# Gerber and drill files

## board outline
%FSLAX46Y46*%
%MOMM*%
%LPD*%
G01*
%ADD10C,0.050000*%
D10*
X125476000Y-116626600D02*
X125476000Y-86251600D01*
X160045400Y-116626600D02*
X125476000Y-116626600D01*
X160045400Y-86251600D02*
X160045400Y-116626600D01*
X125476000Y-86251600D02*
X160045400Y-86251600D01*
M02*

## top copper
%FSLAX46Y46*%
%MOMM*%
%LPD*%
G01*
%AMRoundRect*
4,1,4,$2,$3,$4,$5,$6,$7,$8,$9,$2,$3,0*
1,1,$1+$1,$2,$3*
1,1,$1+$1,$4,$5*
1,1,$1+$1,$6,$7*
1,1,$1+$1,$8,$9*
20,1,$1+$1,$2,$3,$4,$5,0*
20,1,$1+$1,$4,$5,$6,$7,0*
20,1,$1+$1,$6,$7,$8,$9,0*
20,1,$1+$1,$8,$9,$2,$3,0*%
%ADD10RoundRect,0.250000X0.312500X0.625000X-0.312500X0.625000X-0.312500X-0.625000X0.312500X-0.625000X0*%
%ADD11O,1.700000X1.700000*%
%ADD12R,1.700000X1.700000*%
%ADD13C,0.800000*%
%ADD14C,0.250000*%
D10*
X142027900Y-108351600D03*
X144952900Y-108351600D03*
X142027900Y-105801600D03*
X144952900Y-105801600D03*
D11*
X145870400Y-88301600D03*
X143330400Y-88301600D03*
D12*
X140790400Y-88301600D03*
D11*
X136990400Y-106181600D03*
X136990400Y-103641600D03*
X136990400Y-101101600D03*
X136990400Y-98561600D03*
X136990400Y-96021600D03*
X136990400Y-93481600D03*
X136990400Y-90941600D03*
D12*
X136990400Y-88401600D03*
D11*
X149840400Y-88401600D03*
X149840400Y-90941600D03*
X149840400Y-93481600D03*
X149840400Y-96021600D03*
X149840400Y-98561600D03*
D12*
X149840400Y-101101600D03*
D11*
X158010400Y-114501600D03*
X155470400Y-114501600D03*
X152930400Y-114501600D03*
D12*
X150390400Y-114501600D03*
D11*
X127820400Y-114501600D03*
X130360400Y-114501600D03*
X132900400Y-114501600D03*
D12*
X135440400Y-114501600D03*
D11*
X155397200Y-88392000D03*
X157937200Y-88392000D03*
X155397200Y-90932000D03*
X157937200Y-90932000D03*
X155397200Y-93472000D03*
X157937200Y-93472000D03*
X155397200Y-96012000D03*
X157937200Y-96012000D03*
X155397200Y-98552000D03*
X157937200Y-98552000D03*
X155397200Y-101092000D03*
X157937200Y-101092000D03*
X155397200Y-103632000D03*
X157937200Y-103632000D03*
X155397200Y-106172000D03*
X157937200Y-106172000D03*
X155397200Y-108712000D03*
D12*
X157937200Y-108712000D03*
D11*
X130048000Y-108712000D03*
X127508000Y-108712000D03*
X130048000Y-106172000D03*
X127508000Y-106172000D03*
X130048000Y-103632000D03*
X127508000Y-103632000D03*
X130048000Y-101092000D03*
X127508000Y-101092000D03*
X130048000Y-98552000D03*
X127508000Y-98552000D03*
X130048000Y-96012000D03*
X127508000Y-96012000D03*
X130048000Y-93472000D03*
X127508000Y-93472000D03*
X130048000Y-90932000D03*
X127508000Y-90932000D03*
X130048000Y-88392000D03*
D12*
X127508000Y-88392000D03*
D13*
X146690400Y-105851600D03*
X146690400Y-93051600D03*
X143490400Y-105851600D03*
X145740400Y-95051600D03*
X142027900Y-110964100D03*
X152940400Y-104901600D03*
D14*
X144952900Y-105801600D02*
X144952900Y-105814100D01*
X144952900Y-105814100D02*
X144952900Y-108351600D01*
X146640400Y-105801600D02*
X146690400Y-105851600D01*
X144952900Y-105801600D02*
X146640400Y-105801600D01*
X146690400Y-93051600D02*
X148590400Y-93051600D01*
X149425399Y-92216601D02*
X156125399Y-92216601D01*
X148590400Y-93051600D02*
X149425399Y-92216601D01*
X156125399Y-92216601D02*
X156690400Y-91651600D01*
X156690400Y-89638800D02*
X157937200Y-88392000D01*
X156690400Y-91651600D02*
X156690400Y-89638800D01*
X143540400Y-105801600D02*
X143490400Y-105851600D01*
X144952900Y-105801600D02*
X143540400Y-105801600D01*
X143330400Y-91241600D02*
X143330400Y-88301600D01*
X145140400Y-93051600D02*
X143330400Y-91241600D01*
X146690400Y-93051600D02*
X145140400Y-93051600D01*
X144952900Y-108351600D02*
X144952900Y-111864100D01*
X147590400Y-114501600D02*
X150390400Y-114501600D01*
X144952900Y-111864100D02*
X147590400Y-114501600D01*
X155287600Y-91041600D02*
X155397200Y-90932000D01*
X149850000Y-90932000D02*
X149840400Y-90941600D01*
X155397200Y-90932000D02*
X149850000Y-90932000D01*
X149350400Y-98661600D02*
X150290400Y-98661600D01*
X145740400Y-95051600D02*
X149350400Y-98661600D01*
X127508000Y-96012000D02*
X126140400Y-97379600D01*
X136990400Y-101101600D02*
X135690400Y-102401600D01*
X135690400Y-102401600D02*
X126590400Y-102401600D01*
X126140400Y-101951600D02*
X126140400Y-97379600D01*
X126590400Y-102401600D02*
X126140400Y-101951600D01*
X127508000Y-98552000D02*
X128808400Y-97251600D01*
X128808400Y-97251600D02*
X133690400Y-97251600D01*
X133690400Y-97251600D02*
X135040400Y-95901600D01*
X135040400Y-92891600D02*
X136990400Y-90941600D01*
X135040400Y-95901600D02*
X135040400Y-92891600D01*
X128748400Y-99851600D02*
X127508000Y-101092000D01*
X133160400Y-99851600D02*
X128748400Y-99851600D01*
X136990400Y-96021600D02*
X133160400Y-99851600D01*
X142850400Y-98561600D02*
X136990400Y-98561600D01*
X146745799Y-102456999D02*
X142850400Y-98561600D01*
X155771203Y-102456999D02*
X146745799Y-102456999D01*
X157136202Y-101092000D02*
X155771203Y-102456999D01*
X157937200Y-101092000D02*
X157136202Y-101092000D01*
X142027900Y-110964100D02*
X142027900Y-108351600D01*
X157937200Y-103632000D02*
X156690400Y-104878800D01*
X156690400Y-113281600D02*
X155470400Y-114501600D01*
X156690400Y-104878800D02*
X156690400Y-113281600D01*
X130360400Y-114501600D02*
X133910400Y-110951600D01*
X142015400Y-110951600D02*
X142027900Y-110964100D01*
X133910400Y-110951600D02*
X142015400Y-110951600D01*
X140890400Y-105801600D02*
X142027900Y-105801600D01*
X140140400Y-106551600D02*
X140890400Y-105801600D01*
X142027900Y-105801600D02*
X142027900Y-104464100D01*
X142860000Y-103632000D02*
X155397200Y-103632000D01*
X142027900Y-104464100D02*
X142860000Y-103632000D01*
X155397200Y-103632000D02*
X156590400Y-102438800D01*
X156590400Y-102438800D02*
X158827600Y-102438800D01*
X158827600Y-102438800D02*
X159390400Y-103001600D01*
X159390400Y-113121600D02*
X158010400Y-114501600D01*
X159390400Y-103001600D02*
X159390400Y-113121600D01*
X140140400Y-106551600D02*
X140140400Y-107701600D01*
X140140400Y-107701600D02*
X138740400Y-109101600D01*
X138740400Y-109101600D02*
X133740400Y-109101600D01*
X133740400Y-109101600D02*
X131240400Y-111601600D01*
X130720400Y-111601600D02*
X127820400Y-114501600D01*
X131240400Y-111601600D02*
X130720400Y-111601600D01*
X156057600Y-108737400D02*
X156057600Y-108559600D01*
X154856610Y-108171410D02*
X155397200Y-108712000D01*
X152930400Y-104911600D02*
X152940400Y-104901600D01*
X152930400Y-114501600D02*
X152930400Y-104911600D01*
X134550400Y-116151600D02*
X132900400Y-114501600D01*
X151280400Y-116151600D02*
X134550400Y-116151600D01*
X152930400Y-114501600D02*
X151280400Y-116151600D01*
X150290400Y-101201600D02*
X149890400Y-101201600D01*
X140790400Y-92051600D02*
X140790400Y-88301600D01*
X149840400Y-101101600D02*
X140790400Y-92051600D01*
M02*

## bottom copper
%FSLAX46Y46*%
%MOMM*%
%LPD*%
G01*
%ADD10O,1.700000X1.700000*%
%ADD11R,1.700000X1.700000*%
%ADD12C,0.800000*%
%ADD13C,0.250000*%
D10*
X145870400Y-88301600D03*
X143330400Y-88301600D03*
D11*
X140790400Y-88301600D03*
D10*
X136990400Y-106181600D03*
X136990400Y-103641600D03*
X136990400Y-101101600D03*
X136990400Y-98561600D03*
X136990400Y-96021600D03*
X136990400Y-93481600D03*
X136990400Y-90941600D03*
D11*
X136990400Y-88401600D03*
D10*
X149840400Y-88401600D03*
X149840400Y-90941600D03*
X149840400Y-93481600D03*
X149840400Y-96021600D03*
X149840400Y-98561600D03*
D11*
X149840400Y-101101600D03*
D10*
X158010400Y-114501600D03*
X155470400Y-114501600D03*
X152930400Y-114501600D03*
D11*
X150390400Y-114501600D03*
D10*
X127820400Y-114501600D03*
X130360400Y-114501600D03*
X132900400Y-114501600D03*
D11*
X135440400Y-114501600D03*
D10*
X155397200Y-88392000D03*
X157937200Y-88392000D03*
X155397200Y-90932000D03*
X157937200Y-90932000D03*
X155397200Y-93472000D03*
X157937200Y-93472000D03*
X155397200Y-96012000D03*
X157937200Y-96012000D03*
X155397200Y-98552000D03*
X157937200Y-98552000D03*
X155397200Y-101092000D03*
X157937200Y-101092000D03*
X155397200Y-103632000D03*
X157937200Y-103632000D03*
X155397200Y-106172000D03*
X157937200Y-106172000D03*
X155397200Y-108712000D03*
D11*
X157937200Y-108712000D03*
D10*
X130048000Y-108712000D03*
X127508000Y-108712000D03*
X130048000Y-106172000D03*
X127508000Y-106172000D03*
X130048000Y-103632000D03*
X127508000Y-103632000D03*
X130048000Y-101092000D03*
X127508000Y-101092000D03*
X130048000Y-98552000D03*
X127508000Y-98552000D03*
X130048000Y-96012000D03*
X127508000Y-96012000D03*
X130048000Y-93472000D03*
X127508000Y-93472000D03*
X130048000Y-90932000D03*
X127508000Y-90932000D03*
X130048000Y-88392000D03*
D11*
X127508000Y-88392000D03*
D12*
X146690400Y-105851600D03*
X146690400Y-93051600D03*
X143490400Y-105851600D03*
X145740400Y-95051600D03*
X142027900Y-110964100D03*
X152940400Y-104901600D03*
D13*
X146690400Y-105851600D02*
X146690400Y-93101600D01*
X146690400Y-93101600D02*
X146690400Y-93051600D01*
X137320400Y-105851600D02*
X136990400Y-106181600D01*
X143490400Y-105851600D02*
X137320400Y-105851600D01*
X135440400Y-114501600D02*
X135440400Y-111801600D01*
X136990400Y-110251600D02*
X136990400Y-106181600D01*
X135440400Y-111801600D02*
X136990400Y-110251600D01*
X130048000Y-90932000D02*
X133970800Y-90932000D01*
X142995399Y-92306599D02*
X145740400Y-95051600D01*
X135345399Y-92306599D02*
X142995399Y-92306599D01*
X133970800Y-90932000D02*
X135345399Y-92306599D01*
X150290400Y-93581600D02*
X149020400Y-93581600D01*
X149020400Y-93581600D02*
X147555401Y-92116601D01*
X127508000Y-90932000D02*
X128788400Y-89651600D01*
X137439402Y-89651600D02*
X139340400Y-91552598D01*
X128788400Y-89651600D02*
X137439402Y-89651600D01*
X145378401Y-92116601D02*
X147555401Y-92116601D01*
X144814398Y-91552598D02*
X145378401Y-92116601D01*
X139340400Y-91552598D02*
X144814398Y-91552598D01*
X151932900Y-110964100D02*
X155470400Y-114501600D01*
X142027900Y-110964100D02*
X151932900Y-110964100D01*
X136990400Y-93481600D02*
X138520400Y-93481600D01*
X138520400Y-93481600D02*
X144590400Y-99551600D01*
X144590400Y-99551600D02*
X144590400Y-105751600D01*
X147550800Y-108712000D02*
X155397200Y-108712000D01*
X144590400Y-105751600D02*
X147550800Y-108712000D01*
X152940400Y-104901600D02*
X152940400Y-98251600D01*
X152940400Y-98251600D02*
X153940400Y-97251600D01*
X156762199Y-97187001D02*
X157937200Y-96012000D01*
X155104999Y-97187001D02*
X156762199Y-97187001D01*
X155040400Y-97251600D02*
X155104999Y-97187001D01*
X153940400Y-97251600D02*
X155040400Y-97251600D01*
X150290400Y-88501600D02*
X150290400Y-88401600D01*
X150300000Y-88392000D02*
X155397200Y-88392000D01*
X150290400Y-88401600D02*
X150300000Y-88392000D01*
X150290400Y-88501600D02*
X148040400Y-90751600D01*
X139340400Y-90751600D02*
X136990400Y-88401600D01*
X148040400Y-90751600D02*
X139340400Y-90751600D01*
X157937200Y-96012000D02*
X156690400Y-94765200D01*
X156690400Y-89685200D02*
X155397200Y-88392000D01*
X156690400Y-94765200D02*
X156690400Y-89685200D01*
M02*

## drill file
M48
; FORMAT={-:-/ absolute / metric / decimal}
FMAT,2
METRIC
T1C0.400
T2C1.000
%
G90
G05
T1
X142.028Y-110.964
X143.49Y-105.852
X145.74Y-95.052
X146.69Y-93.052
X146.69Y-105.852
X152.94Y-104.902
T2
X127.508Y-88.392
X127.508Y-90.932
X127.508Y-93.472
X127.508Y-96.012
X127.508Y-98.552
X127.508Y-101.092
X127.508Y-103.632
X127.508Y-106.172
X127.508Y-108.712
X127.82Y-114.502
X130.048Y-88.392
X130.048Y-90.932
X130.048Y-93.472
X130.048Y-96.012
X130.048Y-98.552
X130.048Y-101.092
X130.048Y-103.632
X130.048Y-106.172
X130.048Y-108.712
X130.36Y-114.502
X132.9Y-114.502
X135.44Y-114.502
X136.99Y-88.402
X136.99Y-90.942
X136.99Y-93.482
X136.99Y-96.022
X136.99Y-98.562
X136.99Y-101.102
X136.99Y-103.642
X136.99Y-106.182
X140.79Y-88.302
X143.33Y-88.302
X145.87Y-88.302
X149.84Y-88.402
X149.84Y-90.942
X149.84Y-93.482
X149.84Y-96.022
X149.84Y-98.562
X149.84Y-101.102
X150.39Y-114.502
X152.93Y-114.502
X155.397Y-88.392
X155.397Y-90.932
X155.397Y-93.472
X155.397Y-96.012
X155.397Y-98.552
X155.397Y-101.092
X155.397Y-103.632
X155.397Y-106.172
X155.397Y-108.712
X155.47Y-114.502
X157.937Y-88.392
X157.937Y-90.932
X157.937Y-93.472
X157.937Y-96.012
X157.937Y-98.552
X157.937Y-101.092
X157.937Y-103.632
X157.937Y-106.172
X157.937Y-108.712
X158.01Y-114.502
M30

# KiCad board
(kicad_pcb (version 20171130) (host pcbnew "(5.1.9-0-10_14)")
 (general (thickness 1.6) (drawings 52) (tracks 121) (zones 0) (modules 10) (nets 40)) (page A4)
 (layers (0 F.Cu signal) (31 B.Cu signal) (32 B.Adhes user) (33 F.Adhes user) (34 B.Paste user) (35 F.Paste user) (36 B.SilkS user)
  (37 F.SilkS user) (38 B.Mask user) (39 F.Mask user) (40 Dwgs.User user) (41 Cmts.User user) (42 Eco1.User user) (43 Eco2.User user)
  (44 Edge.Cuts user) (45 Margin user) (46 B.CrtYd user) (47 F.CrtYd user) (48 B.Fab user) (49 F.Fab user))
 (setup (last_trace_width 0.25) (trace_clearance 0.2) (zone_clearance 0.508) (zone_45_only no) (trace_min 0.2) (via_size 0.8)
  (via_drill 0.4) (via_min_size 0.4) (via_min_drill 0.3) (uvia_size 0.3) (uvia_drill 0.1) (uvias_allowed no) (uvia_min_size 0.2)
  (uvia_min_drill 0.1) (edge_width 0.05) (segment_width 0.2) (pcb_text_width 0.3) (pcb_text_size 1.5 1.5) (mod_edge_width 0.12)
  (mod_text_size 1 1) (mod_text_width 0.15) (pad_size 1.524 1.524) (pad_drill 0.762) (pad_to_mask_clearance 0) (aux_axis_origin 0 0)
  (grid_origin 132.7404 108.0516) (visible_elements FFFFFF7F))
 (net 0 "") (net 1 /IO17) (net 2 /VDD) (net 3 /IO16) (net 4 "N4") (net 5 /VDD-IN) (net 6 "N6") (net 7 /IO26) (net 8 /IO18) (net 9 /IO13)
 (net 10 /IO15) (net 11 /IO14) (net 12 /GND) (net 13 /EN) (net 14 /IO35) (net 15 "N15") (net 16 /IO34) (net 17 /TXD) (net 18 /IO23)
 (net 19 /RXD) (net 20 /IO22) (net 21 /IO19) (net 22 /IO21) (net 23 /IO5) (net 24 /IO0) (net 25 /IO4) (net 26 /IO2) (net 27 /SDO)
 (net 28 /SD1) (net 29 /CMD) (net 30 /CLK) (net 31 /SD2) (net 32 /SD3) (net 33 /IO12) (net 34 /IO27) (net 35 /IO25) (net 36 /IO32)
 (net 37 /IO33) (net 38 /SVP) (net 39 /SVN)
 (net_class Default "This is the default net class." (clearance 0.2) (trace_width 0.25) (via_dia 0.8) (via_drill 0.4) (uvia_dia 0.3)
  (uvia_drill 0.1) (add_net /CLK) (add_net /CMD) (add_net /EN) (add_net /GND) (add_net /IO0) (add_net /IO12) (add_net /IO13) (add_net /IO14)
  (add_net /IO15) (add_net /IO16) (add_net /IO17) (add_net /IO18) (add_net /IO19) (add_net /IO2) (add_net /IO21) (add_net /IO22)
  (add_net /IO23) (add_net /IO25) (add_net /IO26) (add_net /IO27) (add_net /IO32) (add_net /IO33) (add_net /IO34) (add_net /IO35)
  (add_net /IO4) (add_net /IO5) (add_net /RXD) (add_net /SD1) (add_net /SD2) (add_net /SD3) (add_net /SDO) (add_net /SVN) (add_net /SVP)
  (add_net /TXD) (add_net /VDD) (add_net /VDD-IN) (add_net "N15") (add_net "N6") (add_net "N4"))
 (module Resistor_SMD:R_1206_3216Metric (layer F.Cu) (at 143.4904 108.3516 180)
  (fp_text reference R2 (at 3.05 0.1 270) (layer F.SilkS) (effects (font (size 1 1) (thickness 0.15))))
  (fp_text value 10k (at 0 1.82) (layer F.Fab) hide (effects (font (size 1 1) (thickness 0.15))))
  (pad 2 smd roundrect (at 1.4625 0 180) (size 1.125 1.75) (layers F.Cu F.Paste F.Mask) (roundrect_rratio 0.222222) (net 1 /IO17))
  (pad 1 smd roundrect (at -1.4625 0 180) (size 1.125 1.75) (layers F.Cu F.Paste F.Mask) (roundrect_rratio 0.222222) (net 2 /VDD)))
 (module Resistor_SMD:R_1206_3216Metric (layer F.Cu) (at 143.4904 105.8016 180)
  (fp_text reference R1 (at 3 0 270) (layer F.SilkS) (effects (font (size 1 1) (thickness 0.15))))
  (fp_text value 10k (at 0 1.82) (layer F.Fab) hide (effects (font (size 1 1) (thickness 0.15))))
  (pad 2 smd roundrect (at 1.4625 0 180) (size 1.125 1.75) (layers F.Cu F.Paste F.Mask) (roundrect_rratio 0.222222) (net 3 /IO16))
  (pad 1 smd roundrect (at -1.4625 0 180) (size 1.125 1.75) (layers F.Cu F.Paste F.Mask) (roundrect_rratio 0.222222) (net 2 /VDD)))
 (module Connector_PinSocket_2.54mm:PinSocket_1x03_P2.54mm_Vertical (layer B.Cu) (at 140.7904 88.3016 270)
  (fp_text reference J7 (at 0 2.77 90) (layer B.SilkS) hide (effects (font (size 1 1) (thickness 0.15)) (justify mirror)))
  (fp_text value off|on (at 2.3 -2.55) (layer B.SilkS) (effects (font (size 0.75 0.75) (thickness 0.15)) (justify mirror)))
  (pad 3 thru_hole oval (at 0 -5.08 270) (size 1.7 1.7) (drill 1) (layers *.Cu *.Mask) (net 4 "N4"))
  (pad 2 thru_hole oval (at 0 -2.54 270) (size 1.7 1.7) (drill 1) (layers *.Cu *.Mask) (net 2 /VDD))
  (pad 1 thru_hole rect (at 0 0 270) (size 1.7 1.7) (drill 1) (layers *.Cu *.Mask) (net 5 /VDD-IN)))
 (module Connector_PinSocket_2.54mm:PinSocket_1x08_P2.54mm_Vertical (layer B.Cu) (at 136.9904 88.4016 180)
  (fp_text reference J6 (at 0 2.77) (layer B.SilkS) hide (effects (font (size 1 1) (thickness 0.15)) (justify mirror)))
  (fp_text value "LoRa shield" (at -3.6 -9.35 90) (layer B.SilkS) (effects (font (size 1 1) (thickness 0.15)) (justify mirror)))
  (pad 8 thru_hole oval (at 0 -17.78 180) (size 1.7 1.7) (drill 1) (layers *.Cu *.Mask) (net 2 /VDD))
  (pad 7 thru_hole oval (at 0 -15.24 180) (size 1.7 1.7) (drill 1) (layers *.Cu *.Mask) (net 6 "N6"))
  (pad 6 thru_hole oval (at 0 -12.7 180) (size 1.7 1.7) (drill 1) (layers *.Cu *.Mask) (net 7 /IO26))
  (pad 5 thru_hole oval (at 0 -10.16 180) (size 1.7 1.7) (drill 1) (layers *.Cu *.Mask) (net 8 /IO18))
  (pad 4 thru_hole oval (at 0 -7.62 180) (size 1.7 1.7) (drill 1) (layers *.Cu *.Mask) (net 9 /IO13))
  (pad 3 thru_hole oval (at 0 -5.08 180) (size 1.7 1.7) (drill 1) (layers *.Cu *.Mask) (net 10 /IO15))
  (pad 2 thru_hole oval (at 0 -2.54 180) (size 1.7 1.7) (drill 1) (layers *.Cu *.Mask) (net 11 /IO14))
  (pad 1 thru_hole rect (at 0 0 180) (size 1.7 1.7) (drill 1) (layers *.Cu *.Mask) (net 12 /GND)))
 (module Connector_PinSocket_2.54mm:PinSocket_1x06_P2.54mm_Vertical (layer B.Cu) (at 149.8404 101.1016)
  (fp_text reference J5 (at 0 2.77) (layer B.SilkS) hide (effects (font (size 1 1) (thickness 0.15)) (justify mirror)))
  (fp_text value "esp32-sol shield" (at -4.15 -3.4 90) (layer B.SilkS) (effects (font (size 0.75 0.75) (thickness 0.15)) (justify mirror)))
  (pad 6 thru_hole oval (at 0 -12.7) (size 1.7 1.7) (drill 1) (layers *.Cu *.Mask) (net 12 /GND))
  (pad 5 thru_hole oval (at 0 -10.16) (size 1.7 1.7) (drill 1) (layers *.Cu *.Mask) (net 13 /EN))
  (pad 4 thru_hole oval (at 0 -7.62) (size 1.7 1.7) (drill 1) (layers *.Cu *.Mask) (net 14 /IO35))
  (pad 3 thru_hole oval (at 0 -5.08) (size 1.7 1.7) (drill 1) (layers *.Cu *.Mask) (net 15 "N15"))
  (pad 2 thru_hole oval (at 0 -2.54) (size 1.7 1.7) (drill 1) (layers *.Cu *.Mask) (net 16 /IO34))
  (pad 1 thru_hole rect (at 0 0) (size 1.7 1.7) (drill 1) (layers *.Cu *.Mask) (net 5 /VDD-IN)))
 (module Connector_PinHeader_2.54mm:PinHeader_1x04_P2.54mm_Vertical (layer B.Cu) (at 150.3904 114.5016 270)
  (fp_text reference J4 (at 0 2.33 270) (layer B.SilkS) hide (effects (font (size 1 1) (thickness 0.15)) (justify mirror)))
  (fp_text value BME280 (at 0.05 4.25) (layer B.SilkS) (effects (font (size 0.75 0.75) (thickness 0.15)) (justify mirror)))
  (pad 4 thru_hole oval (at 0 -7.62 270) (size 1.7 1.7) (drill 1) (layers *.Cu *.Mask) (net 3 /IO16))
  (pad 3 thru_hole oval (at 0 -5.08 270) (size 1.7 1.7) (drill 1) (layers *.Cu *.Mask) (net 1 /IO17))
  (pad 2 thru_hole oval (at 0 -2.54 270) (size 1.7 1.7) (drill 1) (layers *.Cu *.Mask) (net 12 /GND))
  (pad 1 thru_hole rect (at 0 0 270) (size 1.7 1.7) (drill 1) (layers *.Cu *.Mask) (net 2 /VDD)))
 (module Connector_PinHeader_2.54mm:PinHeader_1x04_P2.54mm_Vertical (layer B.Cu) (at 135.4404 114.5016 90)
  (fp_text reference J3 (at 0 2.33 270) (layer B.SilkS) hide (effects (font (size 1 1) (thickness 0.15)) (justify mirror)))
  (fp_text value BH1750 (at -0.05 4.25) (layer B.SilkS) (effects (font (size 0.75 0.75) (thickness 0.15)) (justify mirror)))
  (pad 4 thru_hole oval (at 0 -7.62 90) (size 1.7 1.7) (drill 1) (layers *.Cu *.Mask) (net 3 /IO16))
  (pad 3 thru_hole oval (at 0 -5.08 90) (size 1.7 1.7) (drill 1) (layers *.Cu *.Mask) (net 1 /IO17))
  (pad 2 thru_hole oval (at 0 -2.54 90) (size 1.7 1.7) (drill 1) (layers *.Cu *.Mask) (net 12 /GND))
  (pad 1 thru_hole rect (at 0 0 90) (size 1.7 1.7) (drill 1) (layers *.Cu *.Mask) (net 2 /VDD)))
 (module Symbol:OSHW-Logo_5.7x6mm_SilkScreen (layer F.Cu) (at 143.6404 94.9016)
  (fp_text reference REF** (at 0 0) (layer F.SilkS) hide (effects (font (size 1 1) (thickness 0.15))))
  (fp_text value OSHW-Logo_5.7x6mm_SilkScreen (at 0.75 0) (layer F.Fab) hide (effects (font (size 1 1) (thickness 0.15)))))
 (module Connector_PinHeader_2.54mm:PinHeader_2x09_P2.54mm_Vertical (layer F.Cu) (at 157.9372 108.712 180)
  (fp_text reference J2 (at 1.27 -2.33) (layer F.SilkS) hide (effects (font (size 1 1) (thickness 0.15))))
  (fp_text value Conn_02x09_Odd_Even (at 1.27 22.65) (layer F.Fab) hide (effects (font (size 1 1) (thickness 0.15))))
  (pad 18 thru_hole oval (at 2.54 20.32 180) (size 1.7 1.7) (drill 1) (layers *.Cu *.Mask) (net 12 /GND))
  (pad 17 thru_hole oval (at 0 20.32 180) (size 1.7 1.7) (drill 1) (layers *.Cu *.Mask) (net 2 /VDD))
  (pad 16 thru_hole oval (at 2.54 17.78 180) (size 1.7 1.7) (drill 1) (layers *.Cu *.Mask) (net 13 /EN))
  (pad 15 thru_hole oval (at 0 17.78 180) (size 1.7 1.7) (drill 1) (layers *.Cu *.Mask) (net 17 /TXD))
  (pad 14 thru_hole oval (at 2.54 15.24 180) (size 1.7 1.7) (drill 1) (layers *.Cu *.Mask) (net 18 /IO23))
  (pad 13 thru_hole oval (at 0 15.24 180) (size 1.7 1.7) (drill 1) (layers *.Cu *.Mask) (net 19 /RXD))
  (pad 12 thru_hole oval (at 2.54 12.7 180) (size 1.7 1.7) (drill 1) (layers *.Cu *.Mask) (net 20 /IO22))
  (pad 11 thru_hole oval (at 0 12.7 180) (size 1.7 1.7) (drill 1) (layers *.Cu *.Mask) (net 12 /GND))
  (pad 10 thru_hole oval (at 2.54 10.16 180) (size 1.7 1.7) (drill 1) (layers *.Cu *.Mask) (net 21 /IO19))
  (pad 9 thru_hole oval (at 0 10.16 180) (size 1.7 1.7) (drill 1) (layers *.Cu *.Mask) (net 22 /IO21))
  (pad 8 thru_hole oval (at 2.54 7.62 180) (size 1.7 1.7) (drill 1) (layers *.Cu *.Mask) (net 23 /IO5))
  (pad 7 thru_hole oval (at 0 7.62 180) (size 1.7 1.7) (drill 1) (layers *.Cu *.Mask) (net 8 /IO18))
  (pad 6 thru_hole oval (at 2.54 5.08 180) (size 1.7 1.7) (drill 1) (layers *.Cu *.Mask) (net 3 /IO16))
  (pad 5 thru_hole oval (at 0 5.08 180) (size 1.7 1.7) (drill 1) (layers *.Cu *.Mask) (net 1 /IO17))
  (pad 4 thru_hole oval (at 2.54 2.54 180) (size 1.7 1.7) (drill 1) (layers *.Cu *.Mask) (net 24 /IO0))
  (pad 3 thru_hole oval (at 0 2.54 180) (size 1.7 1.7) (drill 1) (layers *.Cu *.Mask) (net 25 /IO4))
  (pad 2 thru_hole oval (at 2.54 0 180) (size 1.7 1.7) (drill 1) (layers *.Cu *.Mask) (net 10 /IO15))
  (pad 1 thru_hole rect (at 0 0 180) (size 1.7 1.7) (drill 1) (layers *.Cu *.Mask) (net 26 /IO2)))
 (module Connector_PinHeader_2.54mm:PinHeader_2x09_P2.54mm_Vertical (layer F.Cu) (at 127.508 88.392)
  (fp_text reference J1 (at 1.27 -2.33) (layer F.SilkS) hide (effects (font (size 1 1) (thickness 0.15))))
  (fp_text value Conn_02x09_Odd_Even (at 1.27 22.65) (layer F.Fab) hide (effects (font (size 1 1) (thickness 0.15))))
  (pad 18 thru_hole oval (at 2.54 20.32) (size 1.7 1.7) (drill 1) (layers *.Cu *.Mask) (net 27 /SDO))
  (pad 17 thru_hole oval (at 0 20.32) (size 1.7 1.7) (drill 1) (layers *.Cu *.Mask) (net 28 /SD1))
  (pad 16 thru_hole oval (at 2.54 17.78) (size 1.7 1.7) (drill 1) (layers *.Cu *.Mask) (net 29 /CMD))
  (pad 15 thru_hole oval (at 0 17.78) (size 1.7 1.7) (drill 1) (layers *.Cu *.Mask) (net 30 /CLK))
  (pad 14 thru_hole oval (at 2.54 15.24) (size 1.7 1.7) (drill 1) (layers *.Cu *.Mask) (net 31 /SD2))
  (pad 13 thru_hole oval (at 0 15.24) (size 1.7 1.7) (drill 1) (layers *.Cu *.Mask) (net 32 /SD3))
  (pad 12 thru_hole oval (at 2.54 12.7) (size 1.7 1.7) (drill 1) (layers *.Cu *.Mask) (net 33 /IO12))
  (pad 11 thru_hole oval (at 0 12.7) (size 1.7 1.7) (drill 1) (layers *.Cu *.Mask) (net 9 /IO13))
  (pad 10 thru_hole oval (at 2.54 10.16) (size 1.7 1.7) (drill 1) (layers *.Cu *.Mask) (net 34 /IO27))
  (pad 9 thru_hole oval (at 0 10.16) (size 1.7 1.7) (drill 1) (layers *.Cu *.Mask) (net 11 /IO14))
  (pad 8 thru_hole oval (at 2.54 7.62) (size 1.7 1.7) (drill 1) (layers *.Cu *.Mask) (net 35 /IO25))
  (pad 7 thru_hole oval (at 0 7.62) (size 1.7 1.7) (drill 1) (layers *.Cu *.Mask) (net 7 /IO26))
  (pad 6 thru_hole oval (at 2.54 5.08) (size 1.7 1.7) (drill 1) (layers *.Cu *.Mask) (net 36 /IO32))
  (pad 5 thru_hole oval (at 0 5.08) (size 1.7 1.7) (drill 1) (layers *.Cu *.Mask) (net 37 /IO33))
  (pad 4 thru_hole oval (at 2.54 2.54) (size 1.7 1.7) (drill 1) (layers *.Cu *.Mask) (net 16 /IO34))
  (pad 3 thru_hole oval (at 0 2.54) (size 1.7 1.7) (drill 1) (layers *.Cu *.Mask) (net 14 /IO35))
  (pad 2 thru_hole oval (at 2.54 0) (size 1.7 1.7) (drill 1) (layers *.Cu *.Mask) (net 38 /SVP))
  (pad 1 thru_hole rect (at 0 0) (size 1.7 1.7) (drill 1) (layers *.Cu *.Mask) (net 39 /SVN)))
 (gr_line (start 125.476 116.6266) (end 125.476 86.2516) (layer Edge.Cuts) (width 0.05))
 (gr_line (start 160.0454 116.6266) (end 125.476 116.6266) (layer Edge.Cuts) (width 0.05))
 (gr_line (start 160.0454 86.2516) (end 160.0454 116.6266) (layer Edge.Cuts) (width 0.05))
 (gr_line (start 125.476 86.2516) (end 160.0454 86.2516) (layer Edge.Cuts) (width 0.05))
 (segment (start 144.9529 105.8016) (end 144.9529 105.8141) (width 0.25) (layer F.Cu) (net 2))
 (segment (start 144.9529 105.8141) (end 144.9529 108.3516) (width 0.25) (layer F.Cu) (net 2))
 (via (at 146.6904 105.8516) (size 0.8) (drill 0.4) (layers F.Cu B.Cu) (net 2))
 (segment (start 146.6404 105.8016) (end 146.6904 105.8516) (width 0.25) (layer F.Cu) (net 2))
 (segment (start 144.9529 105.8016) (end 146.6404 105.8016) (width 0.25) (layer F.Cu) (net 2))
 (segment (start 146.6904 105.8516) (end 146.6904 93.1016) (width 0.25) (layer B.Cu) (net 2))
 (via (at 146.6904 93.0516) (size 0.8) (drill 0.4) (layers F.Cu B.Cu) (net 2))
 (segment (start 146.6904 93.1016) (end 146.6904 93.0516) (width 0.25) (layer B.Cu) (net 2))
 (segment (start 146.6904 93.0516) (end 148.5904 93.0516) (width 0.25) (layer F.Cu) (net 2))
 (segment (start 149.425399 92.216601) (end 156.125399 92.216601) (width 0.25) (layer F.Cu) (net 2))
 (segment (start 148.5904 93.0516) (end 149.425399 92.216601) (width 0.25) (layer F.Cu) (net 2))
 (segment (start 156.125399 92.216601) (end 156.6904 91.6516) (width 0.25) (layer F.Cu) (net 2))
 (segment (start 156.6904 89.6388) (end 157.9372 88.392) (width 0.25) (layer F.Cu) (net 2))
 (segment (start 156.6904 91.6516) (end 156.6904 89.6388) (width 0.25) (layer F.Cu) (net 2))
 (via (at 143.4904 105.8516) (size 0.8) (drill 0.4) (layers F.Cu B.Cu) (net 2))
 (segment (start 143.5404 105.8016) (end 143.4904 105.8516) (width 0.25) (layer F.Cu) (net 2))
 (segment (start 144.9529 105.8016) (end 143.5404 105.8016) (width 0.25) (layer F.Cu) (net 2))
 (segment (start 137.3204 105.8516) (end 136.9904 106.1816) (width 0.25) (layer B.Cu) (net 2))
 (segment (start 143.4904 105.8516) (end 137.3204 105.8516) (width 0.25) (layer B.Cu) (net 2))
 (segment (start 143.3304 91.2416) (end 143.3304 88.3016) (width 0.25) (layer F.Cu) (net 2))
 (segment (start 145.1404 93.0516) (end 143.3304 91.2416) (width 0.25) (layer F.Cu) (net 2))
 (segment (start 146.6904 93.0516) (end 145.1404 93.0516) (width 0.25) (layer F.Cu) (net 2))
 (segment (start 135.4404 114.5016) (end 135.4404 111.8016) (width 0.25) (layer B.Cu) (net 2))
 (segment (start 136.9904 110.2516) (end 136.9904 106.1816) (width 0.25) (layer B.Cu) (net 2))
 (segment (start 135.4404 111.8016) (end 136.9904 110.2516) (width 0.25) (layer B.Cu) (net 2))
 (segment (start 144.9529 108.3516) (end 144.9529 111.8641) (width 0.25) (layer F.Cu) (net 2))
 (segment (start 147.5904 114.5016) (end 150.3904 114.5016) (width 0.25) (layer F.Cu) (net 2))
 (segment (start 144.9529 111.8641) (end 147.5904 114.5016) (width 0.25) (layer F.Cu) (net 2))
 (segment (start 155.2876 91.0416) (end 155.3972 90.932) (width 0.25) (layer F.Cu) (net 13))
 (segment (start 149.85 90.932) (end 149.8404 90.9416) (width 0.25) (layer F.Cu) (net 13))
 (segment (start 155.3972 90.932) (end 149.85 90.932) (width 0.25) (layer F.Cu) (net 13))
 (segment (start 130.048 90.932) (end 133.9708 90.932) (width 0.25) (layer B.Cu) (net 16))
 (via (at 145.7404 95.0516) (size 0.8) (drill 0.4) (layers F.Cu B.Cu) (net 16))
 (segment (start 142.995399 92.306599) (end 145.7404 95.0516) (width 0.25) (layer B.Cu) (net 16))
 (segment (start 135.345399 92.306599) (end 142.995399 92.306599) (width 0.25) (layer B.Cu) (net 16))
 (segment (start 133.9708 90.932) (end 135.345399 92.306599) (width 0.25) (layer B.Cu) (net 16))
 (segment (start 149.3504 98.6616) (end 150.2904 98.6616) (width 0.25) (layer F.Cu) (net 16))
 (segment (start 145.7404 95.0516) (end 149.3504 98.6616) (width 0.25) (layer F.Cu) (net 16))
 (segment (start 150.2904 93.5816) (end 149.0204 93.5816) (width 0.25) (layer B.Cu) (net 14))
 (segment (start 149.0204 93.5816) (end 147.555401 92.116601) (width 0.25) (layer B.Cu) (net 14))
 (segment (start 127.508 90.932) (end 128.7884 89.6516) (width 0.25) (layer B.Cu) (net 14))
 (segment (start 137.439402 89.6516) (end 139.3404 91.552598) (width 0.25) (layer B.Cu) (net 14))
 (segment (start 128.7884 89.6516) (end 137.439402 89.6516) (width 0.25) (layer B.Cu) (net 14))
 (segment (start 145.378401 92.116601) (end 147.555401 92.116601) (width 0.25) (layer B.Cu) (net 14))
 (segment (start 144.814398 91.552598) (end 145.378401 92.116601) (width 0.25) (layer B.Cu) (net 14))
 (segment (start 139.3404 91.552598) (end 144.814398 91.552598) (width 0.25) (layer B.Cu) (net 14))
 (segment (start 127.508 96.012) (end 126.1404 97.3796) (width 0.25) (layer F.Cu) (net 7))
 (segment (start 136.9904 101.1016) (end 135.6904 102.4016) (width 0.25) (layer F.Cu) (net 7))
 (segment (start 135.6904 102.4016) (end 126.5904 102.4016) (width 0.25) (layer F.Cu) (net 7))
 (segment (start 126.1404 101.9516) (end 126.1404 97.3796) (width 0.25) (layer F.Cu) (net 7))
 (segment (start 126.5904 102.4016) (end 126.1404 101.9516) (width 0.25) (layer F.Cu) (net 7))
 (segment (start 127.508 98.552) (end 128.8084 97.2516) (width 0.25) (layer F.Cu) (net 11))
 (segment (start 128.8084 97.2516) (end 133.6904 97.2516) (width 0.25) (layer F.Cu) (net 11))
 (segment (start 133.6904 97.2516) (end 135.0404 95.9016) (width 0.25) (layer F.Cu) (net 11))
 (segment (start 135.0404 92.8916) (end 136.9904 90.9416) (width 0.25) (layer F.Cu) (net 11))
 (segment (start 135.0404 95.9016) (end 135.0404 92.8916) (width 0.25) (layer F.Cu) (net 11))
 (segment (start 128.7484 99.8516) (end 127.508 101.092) (width 0.25) (layer F.Cu) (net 9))
 (segment (start 133.1604 99.8516) (end 128.7484 99.8516) (width 0.25) (layer F.Cu) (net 9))
 (segment (start 136.9904 96.0216) (end 133.1604 99.8516) (width 0.25) (layer F.Cu) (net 9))
 (segment (start 142.8504 98.5616) (end 136.9904 98.5616) (width 0.25) (layer F.Cu) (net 8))
 (segment (start 146.745799 102.456999) (end 142.8504 98.5616) (width 0.25) (layer F.Cu) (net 8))
 (segment (start 155.771203 102.456999) (end 146.745799 102.456999) (width 0.25) (layer F.Cu) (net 8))
 (segment (start 157.136202 101.092) (end 155.771203 102.456999) (width 0.25) (layer F.Cu) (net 8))
 (segment (start 157.9372 101.092) (end 157.136202 101.092) (width 0.25) (layer F.Cu) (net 8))
 (segment (start 142.0279 110.9641) (end 142.0279 108.3516) (width 0.25) (layer F.Cu) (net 1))
 (segment (start 157.9372 103.632) (end 156.6904 104.8788) (width 0.25) (layer F.Cu) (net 1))
 (segment (start 156.6904 113.2816) (end 155.4704 114.5016) (width 0.25) (layer F.Cu) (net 1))
 (segment (start 156.6904 104.8788) (end 156.6904 113.2816) (width 0.25) (layer F.Cu) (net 1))
 (via (at 142.0279 110.9641) (size 0.8) (drill 0.4) (layers F.Cu B.Cu) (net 1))
 (segment (start 151.9329 110.9641) (end 155.4704 114.5016) (width 0.25) (layer B.Cu) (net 1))
 (segment (start 142.0279 110.9641) (end 151.9329 110.9641) (width 0.25) (layer B.Cu) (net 1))
 (segment (start 130.3604 114.5016) (end 133.9104 110.9516) (width 0.25) (layer F.Cu) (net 1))
 (segment (start 142.0154 110.9516) (end 142.0279 110.9641) (width 0.25) (layer F.Cu) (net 1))
 (segment (start 133.9104 110.9516) (end 142.0154 110.9516) (width 0.25) (layer F.Cu) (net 1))
 (segment (start 140.8904 105.8016) (end 142.0279 105.8016) (width 0.25) (layer F.Cu) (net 3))
 (segment (start 140.1404 106.5516) (end 140.8904 105.8016) (width 0.25) (layer F.Cu) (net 3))
 (segment (start 142.0279 105.8016) (end 142.0279 104.4641) (width 0.25) (layer F.Cu) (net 3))
 (segment (start 142.86 103.632) (end 155.3972 103.632) (width 0.25) (layer F.Cu) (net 3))
 (segment (start 142.0279 104.4641) (end 142.86 103.632) (width 0.25) (layer F.Cu) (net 3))
 (segment (start 155.3972 103.632) (end 156.5904 102.4388) (width 0.25) (layer F.Cu) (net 3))
 (segment (start 156.5904 102.4388) (end 158.8276 102.4388) (width 0.25) (layer F.Cu) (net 3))
 (segment (start 158.8276 102.4388) (end 159.3904 103.0016) (width 0.25) (layer F.Cu) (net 3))
 (segment (start 159.3904 113.1216) (end 158.0104 114.5016) (width 0.25) (layer F.Cu) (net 3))
 (segment (start 159.3904 103.0016) (end 159.3904 113.1216) (width 0.25) (layer F.Cu) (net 3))
 (segment (start 140.1404 106.5516) (end 140.1404 107.7016) (width 0.25) (layer F.Cu) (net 3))
 (segment (start 140.1404 107.7016) (end 138.7404 109.1016) (width 0.25) (layer F.Cu) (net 3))
 (segment (start 138.7404 109.1016) (end 133.7404 109.1016) (width 0.25) (layer F.Cu) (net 3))
 (segment (start 133.7404 109.1016) (end 131.2404 111.6016) (width 0.25) (layer F.Cu) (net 3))
 (segment (start 130.7204 111.6016) (end 127.8204 114.5016) (width 0.25) (layer F.Cu) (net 3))
 (segment (start 131.2404 111.6016) (end 130.7204 111.6016) (width 0.25) (layer F.Cu) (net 3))
 (segment (start 156.0576 108.7374) (end 156.0576 108.5596) (width 0.25) (layer F.Cu) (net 10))
 (segment (start 154.85661 108.17141) (end 155.3972 108.712) (width 0.25) (layer F.Cu) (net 10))
 (segment (start 136.9904 93.4816) (end 138.5204 93.4816) (width 0.25) (layer B.Cu) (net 10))
 (segment (start 138.5204 93.4816) (end 144.5904 99.5516) (width 0.25) (layer B.Cu) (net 10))
 (segment (start 144.5904 99.5516) (end 144.5904 105.7516) (width 0.25) (layer B.Cu) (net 10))
 (segment (start 147.5508 108.712) (end 155.3972 108.712) (width 0.25) (layer B.Cu) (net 10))
 (segment (start 144.5904 105.7516) (end 147.5508 108.712) (width 0.25) (layer B.Cu) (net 10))
 (segment (start 152.9304 104.9116) (end 152.9404 104.9016) (width 0.25) (layer F.Cu) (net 12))
 (via (at 152.9404 104.9016) (size 0.8) (drill 0.4) (layers F.Cu B.Cu) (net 12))
 (segment (start 152.9304 114.5016) (end 152.9304 104.9116) (width 0.25) (layer F.Cu) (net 12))
 (segment (start 152.9404 104.9016) (end 152.9404 98.2516) (width 0.25) (layer B.Cu) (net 12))
 (segment (start 152.9404 98.2516) (end 153.9404 97.2516) (width 0.25) (layer B.Cu) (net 12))
 (segment (start 156.762199 97.187001) (end 157.9372 96.012) (width 0.25) (layer B.Cu) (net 12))
 (segment (start 155.104999 97.187001) (end 156.762199 97.187001) (width 0.25) (layer B.Cu) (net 12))
 (segment (start 155.0404 97.2516) (end 155.104999 97.187001) (width 0.25) (layer B.Cu) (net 12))
 (segment (start 153.9404 97.2516) (end 155.0404 97.2516) (width 0.25) (layer B.Cu) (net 12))
 (segment (start 150.2904 88.5016) (end 150.2904 88.4016) (width 0.25) (layer B.Cu) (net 12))
 (segment (start 150.3 88.392) (end 155.3972 88.392) (width 0.25) (layer B.Cu) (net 12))
 (segment (start 150.2904 88.4016) (end 150.3 88.392) (width 0.25) (layer B.Cu) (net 12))
 (segment (start 150.2904 88.5016) (end 148.0404 90.7516) (width 0.25) (layer B.Cu) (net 12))
 (segment (start 139.3404 90.7516) (end 136.9904 88.4016) (width 0.25) (layer B.Cu) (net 12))
 (segment (start 148.0404 90.7516) (end 139.3404 90.7516) (width 0.25) (layer B.Cu) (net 12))
 (segment (start 157.9372 96.012) (end 156.6904 94.7652) (width 0.25) (layer B.Cu) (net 12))
 (segment (start 156.6904 89.6852) (end 155.3972 88.392) (width 0.25) (layer B.Cu) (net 12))
 (segment (start 156.6904 94.7652) (end 156.6904 89.6852) (width 0.25) (layer B.Cu) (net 12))
 (segment (start 134.5504 116.1516) (end 132.9004 114.5016) (width 0.25) (layer F.Cu) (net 12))
 (segment (start 151.2804 116.1516) (end 134.5504 116.1516) (width 0.25) (layer F.Cu) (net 12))
 (segment (start 152.9304 114.5016) (end 151.2804 116.1516) (width 0.25) (layer F.Cu) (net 12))
 (segment (start 150.2904 101.2016) (end 149.8904 101.2016) (width 0.25) (layer F.Cu) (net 5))
 (segment (start 140.7904 92.0516) (end 140.7904 88.3016) (width 0.25) (layer F.Cu) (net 5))
 (segment (start 149.8404 101.1016) (end 140.7904 92.0516) (width 0.25) (layer F.Cu) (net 5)))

